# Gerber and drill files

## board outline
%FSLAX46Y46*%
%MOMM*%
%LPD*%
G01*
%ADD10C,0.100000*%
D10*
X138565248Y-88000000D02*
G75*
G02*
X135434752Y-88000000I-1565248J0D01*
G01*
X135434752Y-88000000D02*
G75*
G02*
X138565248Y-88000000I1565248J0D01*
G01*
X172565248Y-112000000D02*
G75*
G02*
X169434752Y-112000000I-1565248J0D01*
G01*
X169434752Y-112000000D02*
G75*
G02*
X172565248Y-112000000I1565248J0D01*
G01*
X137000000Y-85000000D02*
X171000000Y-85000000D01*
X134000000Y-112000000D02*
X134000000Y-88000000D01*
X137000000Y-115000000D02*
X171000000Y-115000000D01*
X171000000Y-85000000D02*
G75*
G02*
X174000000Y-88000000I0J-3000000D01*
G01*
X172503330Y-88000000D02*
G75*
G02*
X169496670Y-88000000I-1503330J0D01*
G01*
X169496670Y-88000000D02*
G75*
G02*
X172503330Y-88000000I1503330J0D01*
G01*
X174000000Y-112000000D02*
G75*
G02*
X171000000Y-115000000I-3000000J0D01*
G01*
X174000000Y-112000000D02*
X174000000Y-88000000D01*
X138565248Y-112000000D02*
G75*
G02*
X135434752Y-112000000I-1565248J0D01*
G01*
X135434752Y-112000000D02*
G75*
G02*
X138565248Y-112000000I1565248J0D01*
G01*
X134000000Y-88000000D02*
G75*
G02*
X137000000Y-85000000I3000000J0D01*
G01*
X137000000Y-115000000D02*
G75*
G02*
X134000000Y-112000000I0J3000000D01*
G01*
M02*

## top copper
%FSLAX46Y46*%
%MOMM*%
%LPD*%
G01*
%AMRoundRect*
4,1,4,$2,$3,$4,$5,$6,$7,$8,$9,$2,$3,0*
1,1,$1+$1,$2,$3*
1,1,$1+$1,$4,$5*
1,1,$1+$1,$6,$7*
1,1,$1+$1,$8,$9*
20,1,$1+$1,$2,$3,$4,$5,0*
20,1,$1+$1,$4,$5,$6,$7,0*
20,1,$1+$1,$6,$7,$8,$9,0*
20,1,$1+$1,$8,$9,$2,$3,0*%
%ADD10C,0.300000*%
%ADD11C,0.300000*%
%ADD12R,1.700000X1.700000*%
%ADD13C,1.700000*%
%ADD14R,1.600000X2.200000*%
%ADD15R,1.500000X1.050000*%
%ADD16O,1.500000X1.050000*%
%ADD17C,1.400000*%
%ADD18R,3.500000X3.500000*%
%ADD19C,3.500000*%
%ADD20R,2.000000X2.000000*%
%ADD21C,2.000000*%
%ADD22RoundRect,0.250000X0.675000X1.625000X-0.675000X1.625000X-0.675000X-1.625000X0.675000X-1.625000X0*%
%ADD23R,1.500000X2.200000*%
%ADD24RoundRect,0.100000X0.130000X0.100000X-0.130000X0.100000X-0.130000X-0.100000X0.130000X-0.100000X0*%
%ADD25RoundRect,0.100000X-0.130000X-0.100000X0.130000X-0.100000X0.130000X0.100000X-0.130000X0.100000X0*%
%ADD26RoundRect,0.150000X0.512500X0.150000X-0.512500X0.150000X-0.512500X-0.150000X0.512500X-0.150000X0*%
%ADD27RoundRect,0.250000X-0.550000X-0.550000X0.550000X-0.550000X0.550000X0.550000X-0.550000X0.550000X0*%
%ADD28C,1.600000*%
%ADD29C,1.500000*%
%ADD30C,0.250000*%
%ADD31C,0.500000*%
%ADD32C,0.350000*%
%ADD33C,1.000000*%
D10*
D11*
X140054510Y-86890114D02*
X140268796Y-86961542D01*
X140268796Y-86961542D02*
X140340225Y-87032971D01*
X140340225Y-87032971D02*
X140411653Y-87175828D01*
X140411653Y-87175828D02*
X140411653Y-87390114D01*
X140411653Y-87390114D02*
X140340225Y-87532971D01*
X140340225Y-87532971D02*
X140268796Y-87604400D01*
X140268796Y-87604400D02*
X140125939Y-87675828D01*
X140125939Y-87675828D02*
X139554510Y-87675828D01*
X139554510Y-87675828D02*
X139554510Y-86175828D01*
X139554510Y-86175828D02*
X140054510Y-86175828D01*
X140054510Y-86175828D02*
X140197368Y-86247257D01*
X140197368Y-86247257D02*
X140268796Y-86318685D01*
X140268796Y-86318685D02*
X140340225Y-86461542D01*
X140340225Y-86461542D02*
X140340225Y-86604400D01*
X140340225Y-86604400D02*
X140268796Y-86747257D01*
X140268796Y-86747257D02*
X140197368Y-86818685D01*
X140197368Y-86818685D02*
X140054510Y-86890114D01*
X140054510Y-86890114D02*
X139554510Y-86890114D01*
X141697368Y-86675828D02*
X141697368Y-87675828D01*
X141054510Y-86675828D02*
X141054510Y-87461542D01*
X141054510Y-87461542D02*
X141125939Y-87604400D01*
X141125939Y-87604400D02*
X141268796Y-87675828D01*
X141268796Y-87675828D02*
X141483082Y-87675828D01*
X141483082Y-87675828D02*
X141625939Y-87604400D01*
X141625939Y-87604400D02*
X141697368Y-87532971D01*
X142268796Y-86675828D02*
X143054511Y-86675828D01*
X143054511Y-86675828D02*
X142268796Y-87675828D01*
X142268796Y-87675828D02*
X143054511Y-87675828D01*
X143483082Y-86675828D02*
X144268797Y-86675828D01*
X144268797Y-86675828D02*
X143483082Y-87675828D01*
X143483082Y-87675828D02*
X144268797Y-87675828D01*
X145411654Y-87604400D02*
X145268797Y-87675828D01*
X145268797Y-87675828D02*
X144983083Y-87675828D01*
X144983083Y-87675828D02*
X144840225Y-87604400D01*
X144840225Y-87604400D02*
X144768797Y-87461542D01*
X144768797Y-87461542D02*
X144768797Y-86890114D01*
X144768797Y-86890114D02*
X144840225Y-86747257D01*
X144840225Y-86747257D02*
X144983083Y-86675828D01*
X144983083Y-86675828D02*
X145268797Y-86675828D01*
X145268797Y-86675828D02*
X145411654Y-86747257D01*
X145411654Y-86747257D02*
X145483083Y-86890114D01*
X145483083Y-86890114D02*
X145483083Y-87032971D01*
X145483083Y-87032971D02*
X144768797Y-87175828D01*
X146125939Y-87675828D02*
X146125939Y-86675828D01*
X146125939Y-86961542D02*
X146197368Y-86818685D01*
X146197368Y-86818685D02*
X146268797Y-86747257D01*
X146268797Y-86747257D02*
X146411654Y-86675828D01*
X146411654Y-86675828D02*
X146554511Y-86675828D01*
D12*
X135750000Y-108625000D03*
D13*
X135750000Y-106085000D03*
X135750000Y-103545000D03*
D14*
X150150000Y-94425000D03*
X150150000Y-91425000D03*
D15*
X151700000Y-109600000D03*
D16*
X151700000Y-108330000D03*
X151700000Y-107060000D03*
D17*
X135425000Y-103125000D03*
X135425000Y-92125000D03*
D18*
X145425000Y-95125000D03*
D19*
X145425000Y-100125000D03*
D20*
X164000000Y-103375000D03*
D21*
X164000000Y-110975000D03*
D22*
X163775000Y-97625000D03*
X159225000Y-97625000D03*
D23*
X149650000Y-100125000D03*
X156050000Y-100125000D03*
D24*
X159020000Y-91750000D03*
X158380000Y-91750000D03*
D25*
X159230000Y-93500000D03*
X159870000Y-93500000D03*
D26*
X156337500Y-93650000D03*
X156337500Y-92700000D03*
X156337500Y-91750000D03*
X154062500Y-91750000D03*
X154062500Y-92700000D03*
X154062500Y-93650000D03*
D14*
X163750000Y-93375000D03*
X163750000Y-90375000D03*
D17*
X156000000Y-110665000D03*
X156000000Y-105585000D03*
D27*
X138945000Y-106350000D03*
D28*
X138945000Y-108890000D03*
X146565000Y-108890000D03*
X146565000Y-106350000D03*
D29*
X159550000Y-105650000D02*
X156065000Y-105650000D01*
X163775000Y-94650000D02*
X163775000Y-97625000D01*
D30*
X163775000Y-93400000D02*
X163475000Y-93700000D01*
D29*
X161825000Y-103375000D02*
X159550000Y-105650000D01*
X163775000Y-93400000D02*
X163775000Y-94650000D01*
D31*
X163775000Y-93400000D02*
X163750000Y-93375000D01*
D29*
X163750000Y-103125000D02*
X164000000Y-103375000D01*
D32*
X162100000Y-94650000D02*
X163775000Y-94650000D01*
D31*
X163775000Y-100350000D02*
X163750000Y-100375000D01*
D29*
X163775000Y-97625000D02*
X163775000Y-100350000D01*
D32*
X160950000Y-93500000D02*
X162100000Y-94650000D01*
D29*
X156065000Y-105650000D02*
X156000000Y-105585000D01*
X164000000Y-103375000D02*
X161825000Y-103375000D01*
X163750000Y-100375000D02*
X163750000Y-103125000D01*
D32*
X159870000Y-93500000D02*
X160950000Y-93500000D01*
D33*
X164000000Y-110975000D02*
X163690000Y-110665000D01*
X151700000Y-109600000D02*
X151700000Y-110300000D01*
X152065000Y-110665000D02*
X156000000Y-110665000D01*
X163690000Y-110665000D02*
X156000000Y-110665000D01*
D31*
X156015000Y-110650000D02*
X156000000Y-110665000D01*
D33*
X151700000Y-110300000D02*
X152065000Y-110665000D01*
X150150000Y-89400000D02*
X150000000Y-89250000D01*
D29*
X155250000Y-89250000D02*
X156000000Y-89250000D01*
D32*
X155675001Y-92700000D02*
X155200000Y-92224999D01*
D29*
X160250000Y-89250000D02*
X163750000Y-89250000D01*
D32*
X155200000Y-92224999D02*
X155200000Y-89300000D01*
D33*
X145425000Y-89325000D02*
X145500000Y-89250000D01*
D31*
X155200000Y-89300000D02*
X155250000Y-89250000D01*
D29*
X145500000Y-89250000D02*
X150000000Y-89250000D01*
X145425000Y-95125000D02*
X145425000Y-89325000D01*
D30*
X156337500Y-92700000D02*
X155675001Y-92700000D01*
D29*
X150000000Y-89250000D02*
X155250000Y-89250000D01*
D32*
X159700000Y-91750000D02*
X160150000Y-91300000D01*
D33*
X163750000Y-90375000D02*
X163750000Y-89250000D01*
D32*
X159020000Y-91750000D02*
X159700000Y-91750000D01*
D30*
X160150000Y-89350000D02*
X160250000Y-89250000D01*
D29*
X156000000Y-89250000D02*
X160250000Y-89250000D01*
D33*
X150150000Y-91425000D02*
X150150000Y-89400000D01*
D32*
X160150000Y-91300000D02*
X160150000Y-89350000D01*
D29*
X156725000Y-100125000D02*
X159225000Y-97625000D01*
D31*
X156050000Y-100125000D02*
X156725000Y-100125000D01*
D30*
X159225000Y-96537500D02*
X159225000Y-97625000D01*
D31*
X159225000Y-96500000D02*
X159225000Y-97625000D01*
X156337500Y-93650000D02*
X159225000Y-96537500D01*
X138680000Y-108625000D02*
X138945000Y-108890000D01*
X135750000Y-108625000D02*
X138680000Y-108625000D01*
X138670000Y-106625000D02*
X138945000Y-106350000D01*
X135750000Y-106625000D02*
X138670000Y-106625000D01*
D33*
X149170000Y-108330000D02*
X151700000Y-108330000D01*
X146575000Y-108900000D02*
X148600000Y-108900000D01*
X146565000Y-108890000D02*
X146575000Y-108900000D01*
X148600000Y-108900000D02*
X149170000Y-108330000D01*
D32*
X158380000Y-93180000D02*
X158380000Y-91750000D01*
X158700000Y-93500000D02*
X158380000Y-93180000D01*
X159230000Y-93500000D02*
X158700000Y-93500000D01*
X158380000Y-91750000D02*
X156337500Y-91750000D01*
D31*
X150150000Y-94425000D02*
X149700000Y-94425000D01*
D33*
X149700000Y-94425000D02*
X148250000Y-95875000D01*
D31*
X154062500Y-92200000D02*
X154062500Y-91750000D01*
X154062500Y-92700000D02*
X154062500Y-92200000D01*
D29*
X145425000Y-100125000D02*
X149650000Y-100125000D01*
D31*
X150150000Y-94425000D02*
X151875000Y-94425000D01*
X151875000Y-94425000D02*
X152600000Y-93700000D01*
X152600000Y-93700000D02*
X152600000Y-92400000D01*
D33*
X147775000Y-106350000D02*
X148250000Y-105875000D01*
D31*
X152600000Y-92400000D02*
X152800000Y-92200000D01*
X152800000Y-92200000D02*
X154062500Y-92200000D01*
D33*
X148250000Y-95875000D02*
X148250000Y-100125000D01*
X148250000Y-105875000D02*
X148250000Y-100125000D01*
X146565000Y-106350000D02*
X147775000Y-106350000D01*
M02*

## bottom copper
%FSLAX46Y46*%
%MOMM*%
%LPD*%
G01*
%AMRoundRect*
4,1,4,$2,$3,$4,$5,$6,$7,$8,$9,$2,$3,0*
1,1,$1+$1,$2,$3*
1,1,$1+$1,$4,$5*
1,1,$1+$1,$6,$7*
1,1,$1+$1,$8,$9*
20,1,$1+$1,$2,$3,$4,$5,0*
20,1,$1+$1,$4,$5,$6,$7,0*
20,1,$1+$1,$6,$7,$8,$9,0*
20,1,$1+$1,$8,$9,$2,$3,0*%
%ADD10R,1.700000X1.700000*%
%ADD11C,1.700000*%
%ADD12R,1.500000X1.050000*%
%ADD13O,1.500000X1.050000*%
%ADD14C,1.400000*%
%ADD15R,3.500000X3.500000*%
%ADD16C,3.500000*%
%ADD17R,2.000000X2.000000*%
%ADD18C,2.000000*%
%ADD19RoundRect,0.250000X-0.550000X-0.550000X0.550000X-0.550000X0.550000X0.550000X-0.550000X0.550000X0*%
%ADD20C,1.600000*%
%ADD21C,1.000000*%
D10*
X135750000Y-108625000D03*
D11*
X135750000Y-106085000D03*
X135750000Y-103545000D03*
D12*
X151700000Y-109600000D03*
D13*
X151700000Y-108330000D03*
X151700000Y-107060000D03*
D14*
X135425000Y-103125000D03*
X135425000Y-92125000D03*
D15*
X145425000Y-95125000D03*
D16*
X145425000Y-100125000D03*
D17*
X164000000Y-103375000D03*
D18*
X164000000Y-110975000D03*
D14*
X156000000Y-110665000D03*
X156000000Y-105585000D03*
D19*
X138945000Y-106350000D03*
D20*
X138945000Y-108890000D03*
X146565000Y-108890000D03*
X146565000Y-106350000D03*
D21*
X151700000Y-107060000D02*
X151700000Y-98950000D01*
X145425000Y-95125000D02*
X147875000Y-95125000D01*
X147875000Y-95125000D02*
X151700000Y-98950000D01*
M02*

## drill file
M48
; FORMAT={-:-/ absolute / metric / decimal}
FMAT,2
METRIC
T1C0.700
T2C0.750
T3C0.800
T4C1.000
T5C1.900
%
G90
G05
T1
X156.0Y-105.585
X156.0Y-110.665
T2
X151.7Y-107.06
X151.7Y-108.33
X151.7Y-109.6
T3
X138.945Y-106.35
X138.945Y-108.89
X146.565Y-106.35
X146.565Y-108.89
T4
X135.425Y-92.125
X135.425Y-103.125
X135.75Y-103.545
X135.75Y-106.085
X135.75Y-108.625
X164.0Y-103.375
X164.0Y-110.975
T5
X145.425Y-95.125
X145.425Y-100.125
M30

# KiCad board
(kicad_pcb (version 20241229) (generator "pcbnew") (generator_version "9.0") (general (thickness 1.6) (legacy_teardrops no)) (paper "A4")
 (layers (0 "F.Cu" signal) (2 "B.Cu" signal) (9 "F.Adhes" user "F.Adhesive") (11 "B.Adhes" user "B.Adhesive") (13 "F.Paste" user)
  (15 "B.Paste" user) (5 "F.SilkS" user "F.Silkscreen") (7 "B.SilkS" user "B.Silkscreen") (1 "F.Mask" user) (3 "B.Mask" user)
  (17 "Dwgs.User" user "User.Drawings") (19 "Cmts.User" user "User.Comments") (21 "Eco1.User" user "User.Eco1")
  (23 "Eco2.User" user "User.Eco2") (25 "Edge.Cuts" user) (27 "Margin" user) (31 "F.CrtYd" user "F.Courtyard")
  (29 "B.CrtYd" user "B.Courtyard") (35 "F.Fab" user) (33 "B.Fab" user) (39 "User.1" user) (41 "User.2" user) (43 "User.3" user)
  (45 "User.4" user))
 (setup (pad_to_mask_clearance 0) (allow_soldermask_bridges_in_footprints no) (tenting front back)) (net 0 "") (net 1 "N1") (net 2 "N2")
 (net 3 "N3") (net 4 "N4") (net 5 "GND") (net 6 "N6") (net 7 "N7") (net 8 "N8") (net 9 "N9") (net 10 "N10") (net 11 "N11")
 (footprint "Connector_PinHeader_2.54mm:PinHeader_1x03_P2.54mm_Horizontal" (layer "F.Cu") (at 135.75 108.625 180)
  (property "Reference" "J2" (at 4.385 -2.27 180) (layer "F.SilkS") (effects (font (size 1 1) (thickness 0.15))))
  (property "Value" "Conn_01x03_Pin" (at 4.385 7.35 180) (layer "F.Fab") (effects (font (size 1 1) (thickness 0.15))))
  (pad "1" thru_hole rect (at 0 0 180) (size 1.7 1.7) (drill 1) (layers "*.Cu" "*.Mask") (remove_unused_layers no) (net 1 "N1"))
  (pad "2" thru_hole circle (at 0 2.54 180) (size 1.7 1.7) (drill 1) (layers "*.Cu" "*.Mask") (remove_unused_layers no) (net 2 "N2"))
  (pad "3" thru_hole circle (at 0 5.08 180) (size 1.7 1.7) (drill 1) (layers "*.Cu" "*.Mask") (remove_unused_layers no) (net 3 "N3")))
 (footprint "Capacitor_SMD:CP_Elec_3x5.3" (layer "F.Cu") (at 150.15 92.925 90)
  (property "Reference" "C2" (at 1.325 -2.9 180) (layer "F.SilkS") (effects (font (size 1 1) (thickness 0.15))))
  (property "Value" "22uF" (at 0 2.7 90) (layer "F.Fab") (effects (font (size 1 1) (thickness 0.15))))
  (pad "1" smd rect (at -1.5 0 90) (size 2.2 1.6) (layers "F.Cu" "F.Mask" "F.Paste") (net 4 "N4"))
  (pad "2" smd rect (at 1.5 0 90) (size 2.2 1.6) (layers "F.Cu" "F.Mask" "F.Paste") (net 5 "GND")))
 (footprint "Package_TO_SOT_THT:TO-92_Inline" (layer "F.Cu") (at 151.7 109.6 90)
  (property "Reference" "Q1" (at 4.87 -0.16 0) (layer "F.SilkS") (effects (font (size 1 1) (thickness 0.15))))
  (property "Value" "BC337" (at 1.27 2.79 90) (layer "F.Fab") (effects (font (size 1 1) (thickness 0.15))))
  (pad "1" thru_hole rect (at 0 0 90) (size 1.05 1.5) (drill 0.75) (layers "*.Cu" "*.Mask") (remove_unused_layers no) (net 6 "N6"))
  (pad "2" thru_hole oval (at 1.27 0 90) (size 1.05 1.5) (drill 0.75) (layers "*.Cu" "*.Mask") (remove_unused_layers no) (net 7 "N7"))
  (pad "3" thru_hole oval (at 2.54 0 90) (size 1.05 1.5) (drill 0.75) (layers "*.Cu" "*.Mask") (remove_unused_layers no) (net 5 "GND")))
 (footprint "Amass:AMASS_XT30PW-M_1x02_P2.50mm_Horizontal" (layer "F.Cu") (at 145.425 95.125 90)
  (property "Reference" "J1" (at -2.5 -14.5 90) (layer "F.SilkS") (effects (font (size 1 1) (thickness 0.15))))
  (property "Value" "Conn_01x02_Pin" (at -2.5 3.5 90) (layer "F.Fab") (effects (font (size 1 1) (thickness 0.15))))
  (pad "" thru_hole circle (at -8 -10 90) (size 1.4 1.4) (drill 1) (layers "*.Cu" "*.Mask") (remove_unused_layers no))
  (pad "" thru_hole circle (at 3 -10 90) (size 1.4 1.4) (drill 1) (layers "*.Cu" "*.Mask") (remove_unused_layers no))
  (pad "1" thru_hole rect (at 0 0 90) (size 3.5 3.5) (drill 1.9) (layers "*.Cu" "*.Mask") (remove_unused_layers no) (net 5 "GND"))
  (pad "2" thru_hole circle (at -5 0 90) (size 3.5 3.5) (drill 1.9) (layers "*.Cu" "*.Mask") (remove_unused_layers no) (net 4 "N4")))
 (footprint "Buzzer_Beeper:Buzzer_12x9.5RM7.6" (layer "F.Cu") (at 164 103.375 -90)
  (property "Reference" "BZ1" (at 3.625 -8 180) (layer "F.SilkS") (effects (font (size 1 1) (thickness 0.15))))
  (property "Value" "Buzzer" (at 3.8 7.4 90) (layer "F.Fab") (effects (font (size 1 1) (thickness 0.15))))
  (pad "1" thru_hole rect (at 0 0 270) (size 2 2) (drill 1) (layers "*.Cu" "*.Mask") (remove_unused_layers no) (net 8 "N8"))
  (pad "2" thru_hole circle (at 7.6 0 270) (size 2 2) (drill 1) (layers "*.Cu" "*.Mask") (remove_unused_layers no) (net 6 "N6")))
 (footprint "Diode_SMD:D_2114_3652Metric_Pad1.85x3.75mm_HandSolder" (layer "F.Cu") (at 161.5 97.625 180)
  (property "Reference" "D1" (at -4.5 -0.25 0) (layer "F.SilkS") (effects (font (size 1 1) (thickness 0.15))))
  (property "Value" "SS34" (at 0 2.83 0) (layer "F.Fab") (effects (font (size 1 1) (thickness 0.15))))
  (pad "1" smd roundrect (at -2.275 0 180) (size 1.85 3.75) (layers "F.Cu" "F.Mask" "F.Paste") (roundrect_rratio 0.135135) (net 8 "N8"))
  (pad "2" smd roundrect (at 2.275 0 180) (size 1.85 3.75) (layers "F.Cu" "F.Mask" "F.Paste") (roundrect_rratio 0.135135) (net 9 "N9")))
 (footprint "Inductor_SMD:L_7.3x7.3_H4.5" (layer "F.Cu") (at 152.85 100.125)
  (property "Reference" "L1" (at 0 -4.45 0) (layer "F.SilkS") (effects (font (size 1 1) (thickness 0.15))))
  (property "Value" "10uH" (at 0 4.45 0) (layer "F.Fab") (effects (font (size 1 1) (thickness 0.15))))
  (pad "1" smd rect (at -3.2 0) (size 1.5 2.2) (layers "F.Cu" "F.Mask" "F.Paste") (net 4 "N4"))
  (pad "2" smd rect (at 3.2 0) (size 1.5 2.2) (layers "F.Cu" "F.Mask" "F.Paste") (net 9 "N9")))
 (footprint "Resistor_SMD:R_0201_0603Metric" (layer "F.Cu") (at 158.7 91.75 180)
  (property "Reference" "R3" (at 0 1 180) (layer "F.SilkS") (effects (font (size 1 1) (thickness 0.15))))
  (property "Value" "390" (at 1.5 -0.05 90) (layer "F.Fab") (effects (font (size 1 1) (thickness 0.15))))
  (pad "" smd roundrect (at -0.345 0 180) (size 0.318 0.36) (layers "F.Paste") (roundrect_rratio 0.25))
  (pad "" smd roundrect (at 0.345 0 180) (size 0.318 0.36) (layers "F.Paste") (roundrect_rratio 0.25))
  (pad "1" smd roundrect (at -0.32 0 180) (size 0.46 0.4) (layers "F.Cu" "F.Mask") (roundrect_rratio 0.25) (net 5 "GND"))
  (pad "2" smd roundrect (at 0.32 0 180) (size 0.46 0.4) (layers "F.Cu" "F.Mask") (roundrect_rratio 0.25) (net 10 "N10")))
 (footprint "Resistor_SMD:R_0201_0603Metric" (layer "F.Cu") (at 159.55 93.5)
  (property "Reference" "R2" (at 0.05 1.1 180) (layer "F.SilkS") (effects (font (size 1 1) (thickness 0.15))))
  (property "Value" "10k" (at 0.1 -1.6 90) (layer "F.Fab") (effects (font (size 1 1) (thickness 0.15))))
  (pad "" smd roundrect (at -0.345 0) (size 0.318 0.36) (layers "F.Paste") (roundrect_rratio 0.25))
  (pad "" smd roundrect (at 0.345 0) (size 0.318 0.36) (layers "F.Paste") (roundrect_rratio 0.25))
  (pad "1" smd roundrect (at -0.32 0) (size 0.46 0.4) (layers "F.Cu" "F.Mask") (roundrect_rratio 0.25) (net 10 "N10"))
  (pad "2" smd roundrect (at 0.32 0) (size 0.46 0.4) (layers "F.Cu" "F.Mask") (roundrect_rratio 0.25) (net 8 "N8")))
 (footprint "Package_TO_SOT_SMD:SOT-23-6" (layer "F.Cu") (at 155.2 92.7 180)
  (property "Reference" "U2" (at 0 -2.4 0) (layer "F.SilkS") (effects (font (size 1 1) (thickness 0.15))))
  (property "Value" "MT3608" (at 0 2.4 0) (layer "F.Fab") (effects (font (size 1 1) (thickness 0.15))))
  (pad "1" smd roundrect (at -1.1375 -0.95 180) (size 1.325 0.6) (layers "F.Cu" "F.Mask" "F.Paste") (roundrect_rratio 0.25) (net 9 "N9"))
  (pad "2" smd roundrect (at -1.1375 0 180) (size 1.325 0.6) (layers "F.Cu" "F.Mask" "F.Paste") (roundrect_rratio 0.25) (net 5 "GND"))
  (pad "3" smd roundrect (at -1.1375 0.95 180) (size 1.325 0.6) (layers "F.Cu" "F.Mask" "F.Paste") (roundrect_rratio 0.25) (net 10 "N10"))
  (pad "4" smd roundrect (at 1.1375 0.95 180) (size 1.325 0.6) (layers "F.Cu" "F.Mask" "F.Paste") (roundrect_rratio 0.25) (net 4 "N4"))
  (pad "5" smd roundrect (at 1.1375 0 180) (size 1.325 0.6) (layers "F.Cu" "F.Mask" "F.Paste") (roundrect_rratio 0.25) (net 4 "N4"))
  (pad "6" smd roundrect (at 1.1375 -0.95 180) (size 1.325 0.6) (layers "F.Cu" "F.Mask" "F.Paste") (roundrect_rratio 0.25) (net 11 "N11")))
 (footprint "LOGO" (layer "F.Cu") (at 170.25 95.875)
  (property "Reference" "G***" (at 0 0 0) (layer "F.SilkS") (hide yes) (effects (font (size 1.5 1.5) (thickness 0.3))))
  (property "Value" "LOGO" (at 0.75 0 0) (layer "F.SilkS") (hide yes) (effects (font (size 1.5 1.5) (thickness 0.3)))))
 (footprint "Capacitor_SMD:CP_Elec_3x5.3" (layer "F.Cu") (at 163.75 91.875 90)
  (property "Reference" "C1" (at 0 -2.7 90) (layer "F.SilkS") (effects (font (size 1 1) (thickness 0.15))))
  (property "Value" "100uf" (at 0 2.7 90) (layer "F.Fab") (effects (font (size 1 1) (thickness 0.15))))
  (pad "1" smd rect (at -1.5 0 90) (size 2.2 1.6) (layers "F.Cu" "F.Mask" "F.Paste") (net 8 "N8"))
  (pad "2" smd rect (at 1.5 0 90) (size 2.2 1.6) (layers "F.Cu" "F.Mask" "F.Paste") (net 5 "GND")))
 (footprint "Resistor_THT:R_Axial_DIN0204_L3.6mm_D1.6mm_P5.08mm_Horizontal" (layer "F.Cu") (at 156 110.665 90)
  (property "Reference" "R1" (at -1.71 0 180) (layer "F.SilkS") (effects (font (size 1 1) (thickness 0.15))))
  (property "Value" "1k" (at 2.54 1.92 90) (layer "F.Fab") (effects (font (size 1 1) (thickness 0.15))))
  (pad "1" thru_hole circle (at 0 0 90) (size 1.4 1.4) (drill 0.7) (layers "*.Cu" "*.Mask") (remove_unused_layers no) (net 6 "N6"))
  (pad "2" thru_hole circle (at 5.08 0 90) (size 1.4 1.4) (drill 0.7) (layers "*.Cu" "*.Mask") (remove_unused_layers no) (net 8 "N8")))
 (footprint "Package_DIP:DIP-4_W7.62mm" (layer "F.Cu") (at 138.945 106.35)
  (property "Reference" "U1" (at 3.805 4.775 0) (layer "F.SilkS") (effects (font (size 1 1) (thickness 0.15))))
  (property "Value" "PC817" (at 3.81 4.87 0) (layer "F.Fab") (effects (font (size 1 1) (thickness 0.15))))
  (pad "1" thru_hole roundrect (at 0 0) (size 1.6 1.6) (drill 0.8) (layers "*.Cu" "*.Mask") (remove_unused_layers no)
   (roundrect_rratio 0.15625) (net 3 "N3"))
  (pad "2" thru_hole circle (at 0 2.54) (size 1.6 1.6) (drill 0.8) (layers "*.Cu" "*.Mask") (remove_unused_layers no) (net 1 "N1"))
  (pad "3" thru_hole circle (at 7.62 2.54) (size 1.6 1.6) (drill 0.8) (layers "*.Cu" "*.Mask") (remove_unused_layers no) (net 7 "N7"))
  (pad "4" thru_hole circle (at 7.62 0) (size 1.6 1.6) (drill 0.8) (layers "*.Cu" "*.Mask") (remove_unused_layers no) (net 4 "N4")))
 (gr_circle (center 137 88) (end 138.565248 88) (stroke (width 0.1) (type solid)) (fill no) (layer "Edge.Cuts"))
 (gr_circle (center 171 112) (end 172.565248 112) (stroke (width 0.1) (type solid)) (fill no) (layer "Edge.Cuts"))
 (gr_line (start 137 85) (end 171 85) (stroke (width 0.1) (type solid)) (layer "Edge.Cuts"))
 (gr_line (start 134 112) (end 134 88) (stroke (width 0.1) (type solid)) (layer "Edge.Cuts"))
 (gr_line (start 137 115) (end 171 115) (stroke (width 0.1) (type solid)) (layer "Edge.Cuts"))
 (gr_arc (start 171 85) (mid 173.12132 85.87868) (end 174 88) (stroke (width 0.1) (type solid)) (layer "Edge.Cuts"))
 (gr_circle (center 171 88) (end 172.50333 88) (stroke (width 0.1) (type solid)) (fill no) (layer "Edge.Cuts"))
 (gr_arc (start 174 112) (mid 173.12132 114.12132) (end 171 115) (stroke (width 0.1) (type solid)) (layer "Edge.Cuts"))
 (gr_line (start 174 112) (end 174 88) (stroke (width 0.1) (type solid)) (layer "Edge.Cuts"))
 (gr_circle (center 137 112) (end 138.565248 112) (stroke (width 0.1) (type solid)) (fill no) (layer "Edge.Cuts"))
 (gr_arc (start 134 88) (mid 134.87868 85.87868) (end 137 85) (stroke (width 0.1) (type solid)) (layer "Edge.Cuts"))
 (gr_arc (start 137 115) (mid 134.87868 114.12132) (end 134 112) (stroke (width 0.1) (type solid)) (layer "Edge.Cuts"))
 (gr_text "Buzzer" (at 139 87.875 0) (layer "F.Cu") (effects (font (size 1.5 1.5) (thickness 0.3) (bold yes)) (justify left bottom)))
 (segment (start 159.55 105.65) (end 156.065 105.65) (width 1.5) (layer "F.Cu") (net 8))
 (segment (start 163.775 94.65) (end 163.775 97.625) (width 1.5) (layer "F.Cu") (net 8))
 (segment (start 163.775 93.4) (end 163.475 93.7) (width 0.25) (layer "F.Cu") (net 8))
 (segment (start 161.825 103.375) (end 159.55 105.65) (width 1.5) (layer "F.Cu") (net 8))
 (segment (start 163.775 93.4) (end 163.775 94.65) (width 1.5) (layer "F.Cu") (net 8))
 (segment (start 163.775 93.4) (end 163.75 93.375) (width 0.5) (layer "F.Cu") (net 8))
 (segment (start 163.75 103.125) (end 164 103.375) (width 1.5) (layer "F.Cu") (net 8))
 (segment (start 162.1 94.65) (end 163.775 94.65) (width 0.35) (layer "F.Cu") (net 8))
 (segment (start 163.775 100.35) (end 163.75 100.375) (width 0.5) (layer "F.Cu") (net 8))
 (segment (start 163.775 97.625) (end 163.775 100.35) (width 1.5) (layer "F.Cu") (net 8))
 (segment (start 160.95 93.5) (end 162.1 94.65) (width 0.35) (layer "F.Cu") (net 8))
 (segment (start 156.065 105.65) (end 156 105.585) (width 1.5) (layer "F.Cu") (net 8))
 (segment (start 164 103.375) (end 161.825 103.375) (width 1.5) (layer "F.Cu") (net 8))
 (segment (start 163.75 100.375) (end 163.75 103.125) (width 1.5) (layer "F.Cu") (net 8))
 (segment (start 159.87 93.5) (end 160.95 93.5) (width 0.35) (layer "F.Cu") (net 8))
 (segment (start 164 110.975) (end 163.69 110.665) (width 1) (layer "F.Cu") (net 6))
 (segment (start 151.7 109.6) (end 151.7 110.3) (width 1) (layer "F.Cu") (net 6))
 (segment (start 152.065 110.665) (end 156 110.665) (width 1) (layer "F.Cu") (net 6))
 (segment (start 163.69 110.665) (end 156 110.665) (width 1) (layer "F.Cu") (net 6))
 (segment (start 156.015 110.65) (end 156 110.665) (width 0.5) (layer "F.Cu") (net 6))
 (segment (start 151.7 110.3) (end 152.065 110.665) (width 1) (layer "F.Cu") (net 6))
 (segment (start 150.15 89.4) (end 150 89.25) (width 1) (layer "F.Cu") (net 5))
 (segment (start 155.25 89.25) (end 156 89.25) (width 1.5) (layer "F.Cu") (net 5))
 (segment (start 155.675001 92.7) (end 155.2 92.224999) (width 0.35) (layer "F.Cu") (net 5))
 (segment (start 160.25 89.25) (end 163.75 89.25) (width 1.5) (layer "F.Cu") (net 5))
 (segment (start 155.2 92.224999) (end 155.2 89.3) (width 0.35) (layer "F.Cu") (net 5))
 (segment (start 145.425 89.325) (end 145.5 89.25) (width 1) (layer "F.Cu") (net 5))
 (segment (start 155.2 89.3) (end 155.25 89.25) (width 0.5) (layer "F.Cu") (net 5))
 (segment (start 145.5 89.25) (end 150 89.25) (width 1.5) (layer "F.Cu") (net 5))
 (segment (start 145.425 95.125) (end 145.425 89.325) (width 1.5) (layer "F.Cu") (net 5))
 (segment (start 156.3375 92.7) (end 155.675001 92.7) (width 0.25) (layer "F.Cu") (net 5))
 (segment (start 150 89.25) (end 155.25 89.25) (width 1.5) (layer "F.Cu") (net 5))
 (segment (start 159.7 91.75) (end 160.15 91.3) (width 0.35) (layer "F.Cu") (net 5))
 (segment (start 163.75 90.375) (end 163.75 89.25) (width 1) (layer "F.Cu") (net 5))
 (segment (start 159.02 91.75) (end 159.7 91.75) (width 0.35) (layer "F.Cu") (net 5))
 (segment (start 160.15 89.35) (end 160.25 89.25) (width 0.25) (layer "F.Cu") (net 5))
 (segment (start 156 89.25) (end 160.25 89.25) (width 1.5) (layer "F.Cu") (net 5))
 (segment (start 150.15 91.425) (end 150.15 89.4) (width 1) (layer "F.Cu") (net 5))
 (segment (start 160.15 91.3) (end 160.15 89.35) (width 0.35) (layer "F.Cu") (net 5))
 (segment (start 151.7 107.06) (end 151.7 98.95) (width 1) (layer "B.Cu") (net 5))
 (segment (start 145.425 95.125) (end 147.875 95.125) (width 1) (layer "B.Cu") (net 5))
 (segment (start 147.875 95.125) (end 151.7 98.95) (width 1) (layer "B.Cu") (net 5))
 (segment (start 156.725 100.125) (end 159.225 97.625) (width 1.5) (layer "F.Cu") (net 9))
 (segment (start 156.05 100.125) (end 156.725 100.125) (width 0.5) (layer "F.Cu") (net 9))
 (segment (start 159.225 96.5375) (end 159.225 97.625) (width 0.25) (layer "F.Cu") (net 9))
 (segment (start 159.225 96.5) (end 159.225 97.625) (width 0.5) (layer "F.Cu") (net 9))
 (segment (start 156.3375 93.65) (end 159.225 96.5375) (width 0.5) (layer "F.Cu") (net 9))
 (segment (start 138.68 108.625) (end 138.945 108.89) (width 0.5) (layer "F.Cu") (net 1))
 (segment (start 135.75 108.625) (end 138.68 108.625) (width 0.5) (layer "F.Cu") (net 1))
 (segment (start 138.67 106.625) (end 138.945 106.35) (width 0.5) (layer "F.Cu") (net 3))
 (segment (start 135.75 106.625) (end 138.67 106.625) (width 0.5) (layer "F.Cu") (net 3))
 (segment (start 149.17 108.33) (end 151.7 108.33) (width 1) (layer "F.Cu") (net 7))
 (segment (start 146.575 108.9) (end 148.6 108.9) (width 1) (layer "F.Cu") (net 7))
 (segment (start 146.565 108.89) (end 146.575 108.9) (width 1) (layer "F.Cu") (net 7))
 (segment (start 148.6 108.9) (end 149.17 108.33) (width 1) (layer "F.Cu") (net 7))
 (segment (start 158.38 93.18) (end 158.38 91.75) (width 0.35) (layer "F.Cu") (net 10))
 (segment (start 158.7 93.5) (end 158.38 93.18) (width 0.35) (layer "F.Cu") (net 10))
 (segment (start 159.23 93.5) (end 158.7 93.5) (width 0.35) (layer "F.Cu") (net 10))
 (segment (start 158.38 91.75) (end 156.3375 91.75) (width 0.35) (layer "F.Cu") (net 10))
 (segment (start 150.15 94.425) (end 149.7 94.425) (width 0.5) (layer "F.Cu") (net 4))
 (segment (start 149.7 94.425) (end 148.25 95.875) (width 1) (layer "F.Cu") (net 4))
 (segment (start 154.0625 92.2) (end 154.0625 91.75) (width 0.5) (layer "F.Cu") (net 4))
 (segment (start 154.0625 92.7) (end 154.0625 92.2) (width 0.5) (layer "F.Cu") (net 4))
 (segment (start 145.425 100.125) (end 149.65 100.125) (width 1.5) (layer "F.Cu") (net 4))
 (segment (start 150.15 94.425) (end 151.875 94.425) (width 0.5) (layer "F.Cu") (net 4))
 (segment (start 151.875 94.425) (end 152.6 93.7) (width 0.5) (layer "F.Cu") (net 4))
 (segment (start 152.6 93.7) (end 152.6 92.4) (width 0.5) (layer "F.Cu") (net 4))
 (segment (start 147.775 106.35) (end 148.25 105.875) (width 1) (layer "F.Cu") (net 4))
 (segment (start 152.6 92.4) (end 152.8 92.2) (width 0.5) (layer "F.Cu") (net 4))
 (segment (start 152.8 92.2) (end 154.0625 92.2) (width 0.5) (layer "F.Cu") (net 4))
 (segment (start 148.25 95.875) (end 148.25 100.125) (width 1) (layer "F.Cu") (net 4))
 (segment (start 148.25 105.875) (end 148.25 100.125) (width 1) (layer "F.Cu") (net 4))
 (segment (start 146.565 106.35) (end 147.775 106.35) (width 1) (layer "F.Cu") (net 4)))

